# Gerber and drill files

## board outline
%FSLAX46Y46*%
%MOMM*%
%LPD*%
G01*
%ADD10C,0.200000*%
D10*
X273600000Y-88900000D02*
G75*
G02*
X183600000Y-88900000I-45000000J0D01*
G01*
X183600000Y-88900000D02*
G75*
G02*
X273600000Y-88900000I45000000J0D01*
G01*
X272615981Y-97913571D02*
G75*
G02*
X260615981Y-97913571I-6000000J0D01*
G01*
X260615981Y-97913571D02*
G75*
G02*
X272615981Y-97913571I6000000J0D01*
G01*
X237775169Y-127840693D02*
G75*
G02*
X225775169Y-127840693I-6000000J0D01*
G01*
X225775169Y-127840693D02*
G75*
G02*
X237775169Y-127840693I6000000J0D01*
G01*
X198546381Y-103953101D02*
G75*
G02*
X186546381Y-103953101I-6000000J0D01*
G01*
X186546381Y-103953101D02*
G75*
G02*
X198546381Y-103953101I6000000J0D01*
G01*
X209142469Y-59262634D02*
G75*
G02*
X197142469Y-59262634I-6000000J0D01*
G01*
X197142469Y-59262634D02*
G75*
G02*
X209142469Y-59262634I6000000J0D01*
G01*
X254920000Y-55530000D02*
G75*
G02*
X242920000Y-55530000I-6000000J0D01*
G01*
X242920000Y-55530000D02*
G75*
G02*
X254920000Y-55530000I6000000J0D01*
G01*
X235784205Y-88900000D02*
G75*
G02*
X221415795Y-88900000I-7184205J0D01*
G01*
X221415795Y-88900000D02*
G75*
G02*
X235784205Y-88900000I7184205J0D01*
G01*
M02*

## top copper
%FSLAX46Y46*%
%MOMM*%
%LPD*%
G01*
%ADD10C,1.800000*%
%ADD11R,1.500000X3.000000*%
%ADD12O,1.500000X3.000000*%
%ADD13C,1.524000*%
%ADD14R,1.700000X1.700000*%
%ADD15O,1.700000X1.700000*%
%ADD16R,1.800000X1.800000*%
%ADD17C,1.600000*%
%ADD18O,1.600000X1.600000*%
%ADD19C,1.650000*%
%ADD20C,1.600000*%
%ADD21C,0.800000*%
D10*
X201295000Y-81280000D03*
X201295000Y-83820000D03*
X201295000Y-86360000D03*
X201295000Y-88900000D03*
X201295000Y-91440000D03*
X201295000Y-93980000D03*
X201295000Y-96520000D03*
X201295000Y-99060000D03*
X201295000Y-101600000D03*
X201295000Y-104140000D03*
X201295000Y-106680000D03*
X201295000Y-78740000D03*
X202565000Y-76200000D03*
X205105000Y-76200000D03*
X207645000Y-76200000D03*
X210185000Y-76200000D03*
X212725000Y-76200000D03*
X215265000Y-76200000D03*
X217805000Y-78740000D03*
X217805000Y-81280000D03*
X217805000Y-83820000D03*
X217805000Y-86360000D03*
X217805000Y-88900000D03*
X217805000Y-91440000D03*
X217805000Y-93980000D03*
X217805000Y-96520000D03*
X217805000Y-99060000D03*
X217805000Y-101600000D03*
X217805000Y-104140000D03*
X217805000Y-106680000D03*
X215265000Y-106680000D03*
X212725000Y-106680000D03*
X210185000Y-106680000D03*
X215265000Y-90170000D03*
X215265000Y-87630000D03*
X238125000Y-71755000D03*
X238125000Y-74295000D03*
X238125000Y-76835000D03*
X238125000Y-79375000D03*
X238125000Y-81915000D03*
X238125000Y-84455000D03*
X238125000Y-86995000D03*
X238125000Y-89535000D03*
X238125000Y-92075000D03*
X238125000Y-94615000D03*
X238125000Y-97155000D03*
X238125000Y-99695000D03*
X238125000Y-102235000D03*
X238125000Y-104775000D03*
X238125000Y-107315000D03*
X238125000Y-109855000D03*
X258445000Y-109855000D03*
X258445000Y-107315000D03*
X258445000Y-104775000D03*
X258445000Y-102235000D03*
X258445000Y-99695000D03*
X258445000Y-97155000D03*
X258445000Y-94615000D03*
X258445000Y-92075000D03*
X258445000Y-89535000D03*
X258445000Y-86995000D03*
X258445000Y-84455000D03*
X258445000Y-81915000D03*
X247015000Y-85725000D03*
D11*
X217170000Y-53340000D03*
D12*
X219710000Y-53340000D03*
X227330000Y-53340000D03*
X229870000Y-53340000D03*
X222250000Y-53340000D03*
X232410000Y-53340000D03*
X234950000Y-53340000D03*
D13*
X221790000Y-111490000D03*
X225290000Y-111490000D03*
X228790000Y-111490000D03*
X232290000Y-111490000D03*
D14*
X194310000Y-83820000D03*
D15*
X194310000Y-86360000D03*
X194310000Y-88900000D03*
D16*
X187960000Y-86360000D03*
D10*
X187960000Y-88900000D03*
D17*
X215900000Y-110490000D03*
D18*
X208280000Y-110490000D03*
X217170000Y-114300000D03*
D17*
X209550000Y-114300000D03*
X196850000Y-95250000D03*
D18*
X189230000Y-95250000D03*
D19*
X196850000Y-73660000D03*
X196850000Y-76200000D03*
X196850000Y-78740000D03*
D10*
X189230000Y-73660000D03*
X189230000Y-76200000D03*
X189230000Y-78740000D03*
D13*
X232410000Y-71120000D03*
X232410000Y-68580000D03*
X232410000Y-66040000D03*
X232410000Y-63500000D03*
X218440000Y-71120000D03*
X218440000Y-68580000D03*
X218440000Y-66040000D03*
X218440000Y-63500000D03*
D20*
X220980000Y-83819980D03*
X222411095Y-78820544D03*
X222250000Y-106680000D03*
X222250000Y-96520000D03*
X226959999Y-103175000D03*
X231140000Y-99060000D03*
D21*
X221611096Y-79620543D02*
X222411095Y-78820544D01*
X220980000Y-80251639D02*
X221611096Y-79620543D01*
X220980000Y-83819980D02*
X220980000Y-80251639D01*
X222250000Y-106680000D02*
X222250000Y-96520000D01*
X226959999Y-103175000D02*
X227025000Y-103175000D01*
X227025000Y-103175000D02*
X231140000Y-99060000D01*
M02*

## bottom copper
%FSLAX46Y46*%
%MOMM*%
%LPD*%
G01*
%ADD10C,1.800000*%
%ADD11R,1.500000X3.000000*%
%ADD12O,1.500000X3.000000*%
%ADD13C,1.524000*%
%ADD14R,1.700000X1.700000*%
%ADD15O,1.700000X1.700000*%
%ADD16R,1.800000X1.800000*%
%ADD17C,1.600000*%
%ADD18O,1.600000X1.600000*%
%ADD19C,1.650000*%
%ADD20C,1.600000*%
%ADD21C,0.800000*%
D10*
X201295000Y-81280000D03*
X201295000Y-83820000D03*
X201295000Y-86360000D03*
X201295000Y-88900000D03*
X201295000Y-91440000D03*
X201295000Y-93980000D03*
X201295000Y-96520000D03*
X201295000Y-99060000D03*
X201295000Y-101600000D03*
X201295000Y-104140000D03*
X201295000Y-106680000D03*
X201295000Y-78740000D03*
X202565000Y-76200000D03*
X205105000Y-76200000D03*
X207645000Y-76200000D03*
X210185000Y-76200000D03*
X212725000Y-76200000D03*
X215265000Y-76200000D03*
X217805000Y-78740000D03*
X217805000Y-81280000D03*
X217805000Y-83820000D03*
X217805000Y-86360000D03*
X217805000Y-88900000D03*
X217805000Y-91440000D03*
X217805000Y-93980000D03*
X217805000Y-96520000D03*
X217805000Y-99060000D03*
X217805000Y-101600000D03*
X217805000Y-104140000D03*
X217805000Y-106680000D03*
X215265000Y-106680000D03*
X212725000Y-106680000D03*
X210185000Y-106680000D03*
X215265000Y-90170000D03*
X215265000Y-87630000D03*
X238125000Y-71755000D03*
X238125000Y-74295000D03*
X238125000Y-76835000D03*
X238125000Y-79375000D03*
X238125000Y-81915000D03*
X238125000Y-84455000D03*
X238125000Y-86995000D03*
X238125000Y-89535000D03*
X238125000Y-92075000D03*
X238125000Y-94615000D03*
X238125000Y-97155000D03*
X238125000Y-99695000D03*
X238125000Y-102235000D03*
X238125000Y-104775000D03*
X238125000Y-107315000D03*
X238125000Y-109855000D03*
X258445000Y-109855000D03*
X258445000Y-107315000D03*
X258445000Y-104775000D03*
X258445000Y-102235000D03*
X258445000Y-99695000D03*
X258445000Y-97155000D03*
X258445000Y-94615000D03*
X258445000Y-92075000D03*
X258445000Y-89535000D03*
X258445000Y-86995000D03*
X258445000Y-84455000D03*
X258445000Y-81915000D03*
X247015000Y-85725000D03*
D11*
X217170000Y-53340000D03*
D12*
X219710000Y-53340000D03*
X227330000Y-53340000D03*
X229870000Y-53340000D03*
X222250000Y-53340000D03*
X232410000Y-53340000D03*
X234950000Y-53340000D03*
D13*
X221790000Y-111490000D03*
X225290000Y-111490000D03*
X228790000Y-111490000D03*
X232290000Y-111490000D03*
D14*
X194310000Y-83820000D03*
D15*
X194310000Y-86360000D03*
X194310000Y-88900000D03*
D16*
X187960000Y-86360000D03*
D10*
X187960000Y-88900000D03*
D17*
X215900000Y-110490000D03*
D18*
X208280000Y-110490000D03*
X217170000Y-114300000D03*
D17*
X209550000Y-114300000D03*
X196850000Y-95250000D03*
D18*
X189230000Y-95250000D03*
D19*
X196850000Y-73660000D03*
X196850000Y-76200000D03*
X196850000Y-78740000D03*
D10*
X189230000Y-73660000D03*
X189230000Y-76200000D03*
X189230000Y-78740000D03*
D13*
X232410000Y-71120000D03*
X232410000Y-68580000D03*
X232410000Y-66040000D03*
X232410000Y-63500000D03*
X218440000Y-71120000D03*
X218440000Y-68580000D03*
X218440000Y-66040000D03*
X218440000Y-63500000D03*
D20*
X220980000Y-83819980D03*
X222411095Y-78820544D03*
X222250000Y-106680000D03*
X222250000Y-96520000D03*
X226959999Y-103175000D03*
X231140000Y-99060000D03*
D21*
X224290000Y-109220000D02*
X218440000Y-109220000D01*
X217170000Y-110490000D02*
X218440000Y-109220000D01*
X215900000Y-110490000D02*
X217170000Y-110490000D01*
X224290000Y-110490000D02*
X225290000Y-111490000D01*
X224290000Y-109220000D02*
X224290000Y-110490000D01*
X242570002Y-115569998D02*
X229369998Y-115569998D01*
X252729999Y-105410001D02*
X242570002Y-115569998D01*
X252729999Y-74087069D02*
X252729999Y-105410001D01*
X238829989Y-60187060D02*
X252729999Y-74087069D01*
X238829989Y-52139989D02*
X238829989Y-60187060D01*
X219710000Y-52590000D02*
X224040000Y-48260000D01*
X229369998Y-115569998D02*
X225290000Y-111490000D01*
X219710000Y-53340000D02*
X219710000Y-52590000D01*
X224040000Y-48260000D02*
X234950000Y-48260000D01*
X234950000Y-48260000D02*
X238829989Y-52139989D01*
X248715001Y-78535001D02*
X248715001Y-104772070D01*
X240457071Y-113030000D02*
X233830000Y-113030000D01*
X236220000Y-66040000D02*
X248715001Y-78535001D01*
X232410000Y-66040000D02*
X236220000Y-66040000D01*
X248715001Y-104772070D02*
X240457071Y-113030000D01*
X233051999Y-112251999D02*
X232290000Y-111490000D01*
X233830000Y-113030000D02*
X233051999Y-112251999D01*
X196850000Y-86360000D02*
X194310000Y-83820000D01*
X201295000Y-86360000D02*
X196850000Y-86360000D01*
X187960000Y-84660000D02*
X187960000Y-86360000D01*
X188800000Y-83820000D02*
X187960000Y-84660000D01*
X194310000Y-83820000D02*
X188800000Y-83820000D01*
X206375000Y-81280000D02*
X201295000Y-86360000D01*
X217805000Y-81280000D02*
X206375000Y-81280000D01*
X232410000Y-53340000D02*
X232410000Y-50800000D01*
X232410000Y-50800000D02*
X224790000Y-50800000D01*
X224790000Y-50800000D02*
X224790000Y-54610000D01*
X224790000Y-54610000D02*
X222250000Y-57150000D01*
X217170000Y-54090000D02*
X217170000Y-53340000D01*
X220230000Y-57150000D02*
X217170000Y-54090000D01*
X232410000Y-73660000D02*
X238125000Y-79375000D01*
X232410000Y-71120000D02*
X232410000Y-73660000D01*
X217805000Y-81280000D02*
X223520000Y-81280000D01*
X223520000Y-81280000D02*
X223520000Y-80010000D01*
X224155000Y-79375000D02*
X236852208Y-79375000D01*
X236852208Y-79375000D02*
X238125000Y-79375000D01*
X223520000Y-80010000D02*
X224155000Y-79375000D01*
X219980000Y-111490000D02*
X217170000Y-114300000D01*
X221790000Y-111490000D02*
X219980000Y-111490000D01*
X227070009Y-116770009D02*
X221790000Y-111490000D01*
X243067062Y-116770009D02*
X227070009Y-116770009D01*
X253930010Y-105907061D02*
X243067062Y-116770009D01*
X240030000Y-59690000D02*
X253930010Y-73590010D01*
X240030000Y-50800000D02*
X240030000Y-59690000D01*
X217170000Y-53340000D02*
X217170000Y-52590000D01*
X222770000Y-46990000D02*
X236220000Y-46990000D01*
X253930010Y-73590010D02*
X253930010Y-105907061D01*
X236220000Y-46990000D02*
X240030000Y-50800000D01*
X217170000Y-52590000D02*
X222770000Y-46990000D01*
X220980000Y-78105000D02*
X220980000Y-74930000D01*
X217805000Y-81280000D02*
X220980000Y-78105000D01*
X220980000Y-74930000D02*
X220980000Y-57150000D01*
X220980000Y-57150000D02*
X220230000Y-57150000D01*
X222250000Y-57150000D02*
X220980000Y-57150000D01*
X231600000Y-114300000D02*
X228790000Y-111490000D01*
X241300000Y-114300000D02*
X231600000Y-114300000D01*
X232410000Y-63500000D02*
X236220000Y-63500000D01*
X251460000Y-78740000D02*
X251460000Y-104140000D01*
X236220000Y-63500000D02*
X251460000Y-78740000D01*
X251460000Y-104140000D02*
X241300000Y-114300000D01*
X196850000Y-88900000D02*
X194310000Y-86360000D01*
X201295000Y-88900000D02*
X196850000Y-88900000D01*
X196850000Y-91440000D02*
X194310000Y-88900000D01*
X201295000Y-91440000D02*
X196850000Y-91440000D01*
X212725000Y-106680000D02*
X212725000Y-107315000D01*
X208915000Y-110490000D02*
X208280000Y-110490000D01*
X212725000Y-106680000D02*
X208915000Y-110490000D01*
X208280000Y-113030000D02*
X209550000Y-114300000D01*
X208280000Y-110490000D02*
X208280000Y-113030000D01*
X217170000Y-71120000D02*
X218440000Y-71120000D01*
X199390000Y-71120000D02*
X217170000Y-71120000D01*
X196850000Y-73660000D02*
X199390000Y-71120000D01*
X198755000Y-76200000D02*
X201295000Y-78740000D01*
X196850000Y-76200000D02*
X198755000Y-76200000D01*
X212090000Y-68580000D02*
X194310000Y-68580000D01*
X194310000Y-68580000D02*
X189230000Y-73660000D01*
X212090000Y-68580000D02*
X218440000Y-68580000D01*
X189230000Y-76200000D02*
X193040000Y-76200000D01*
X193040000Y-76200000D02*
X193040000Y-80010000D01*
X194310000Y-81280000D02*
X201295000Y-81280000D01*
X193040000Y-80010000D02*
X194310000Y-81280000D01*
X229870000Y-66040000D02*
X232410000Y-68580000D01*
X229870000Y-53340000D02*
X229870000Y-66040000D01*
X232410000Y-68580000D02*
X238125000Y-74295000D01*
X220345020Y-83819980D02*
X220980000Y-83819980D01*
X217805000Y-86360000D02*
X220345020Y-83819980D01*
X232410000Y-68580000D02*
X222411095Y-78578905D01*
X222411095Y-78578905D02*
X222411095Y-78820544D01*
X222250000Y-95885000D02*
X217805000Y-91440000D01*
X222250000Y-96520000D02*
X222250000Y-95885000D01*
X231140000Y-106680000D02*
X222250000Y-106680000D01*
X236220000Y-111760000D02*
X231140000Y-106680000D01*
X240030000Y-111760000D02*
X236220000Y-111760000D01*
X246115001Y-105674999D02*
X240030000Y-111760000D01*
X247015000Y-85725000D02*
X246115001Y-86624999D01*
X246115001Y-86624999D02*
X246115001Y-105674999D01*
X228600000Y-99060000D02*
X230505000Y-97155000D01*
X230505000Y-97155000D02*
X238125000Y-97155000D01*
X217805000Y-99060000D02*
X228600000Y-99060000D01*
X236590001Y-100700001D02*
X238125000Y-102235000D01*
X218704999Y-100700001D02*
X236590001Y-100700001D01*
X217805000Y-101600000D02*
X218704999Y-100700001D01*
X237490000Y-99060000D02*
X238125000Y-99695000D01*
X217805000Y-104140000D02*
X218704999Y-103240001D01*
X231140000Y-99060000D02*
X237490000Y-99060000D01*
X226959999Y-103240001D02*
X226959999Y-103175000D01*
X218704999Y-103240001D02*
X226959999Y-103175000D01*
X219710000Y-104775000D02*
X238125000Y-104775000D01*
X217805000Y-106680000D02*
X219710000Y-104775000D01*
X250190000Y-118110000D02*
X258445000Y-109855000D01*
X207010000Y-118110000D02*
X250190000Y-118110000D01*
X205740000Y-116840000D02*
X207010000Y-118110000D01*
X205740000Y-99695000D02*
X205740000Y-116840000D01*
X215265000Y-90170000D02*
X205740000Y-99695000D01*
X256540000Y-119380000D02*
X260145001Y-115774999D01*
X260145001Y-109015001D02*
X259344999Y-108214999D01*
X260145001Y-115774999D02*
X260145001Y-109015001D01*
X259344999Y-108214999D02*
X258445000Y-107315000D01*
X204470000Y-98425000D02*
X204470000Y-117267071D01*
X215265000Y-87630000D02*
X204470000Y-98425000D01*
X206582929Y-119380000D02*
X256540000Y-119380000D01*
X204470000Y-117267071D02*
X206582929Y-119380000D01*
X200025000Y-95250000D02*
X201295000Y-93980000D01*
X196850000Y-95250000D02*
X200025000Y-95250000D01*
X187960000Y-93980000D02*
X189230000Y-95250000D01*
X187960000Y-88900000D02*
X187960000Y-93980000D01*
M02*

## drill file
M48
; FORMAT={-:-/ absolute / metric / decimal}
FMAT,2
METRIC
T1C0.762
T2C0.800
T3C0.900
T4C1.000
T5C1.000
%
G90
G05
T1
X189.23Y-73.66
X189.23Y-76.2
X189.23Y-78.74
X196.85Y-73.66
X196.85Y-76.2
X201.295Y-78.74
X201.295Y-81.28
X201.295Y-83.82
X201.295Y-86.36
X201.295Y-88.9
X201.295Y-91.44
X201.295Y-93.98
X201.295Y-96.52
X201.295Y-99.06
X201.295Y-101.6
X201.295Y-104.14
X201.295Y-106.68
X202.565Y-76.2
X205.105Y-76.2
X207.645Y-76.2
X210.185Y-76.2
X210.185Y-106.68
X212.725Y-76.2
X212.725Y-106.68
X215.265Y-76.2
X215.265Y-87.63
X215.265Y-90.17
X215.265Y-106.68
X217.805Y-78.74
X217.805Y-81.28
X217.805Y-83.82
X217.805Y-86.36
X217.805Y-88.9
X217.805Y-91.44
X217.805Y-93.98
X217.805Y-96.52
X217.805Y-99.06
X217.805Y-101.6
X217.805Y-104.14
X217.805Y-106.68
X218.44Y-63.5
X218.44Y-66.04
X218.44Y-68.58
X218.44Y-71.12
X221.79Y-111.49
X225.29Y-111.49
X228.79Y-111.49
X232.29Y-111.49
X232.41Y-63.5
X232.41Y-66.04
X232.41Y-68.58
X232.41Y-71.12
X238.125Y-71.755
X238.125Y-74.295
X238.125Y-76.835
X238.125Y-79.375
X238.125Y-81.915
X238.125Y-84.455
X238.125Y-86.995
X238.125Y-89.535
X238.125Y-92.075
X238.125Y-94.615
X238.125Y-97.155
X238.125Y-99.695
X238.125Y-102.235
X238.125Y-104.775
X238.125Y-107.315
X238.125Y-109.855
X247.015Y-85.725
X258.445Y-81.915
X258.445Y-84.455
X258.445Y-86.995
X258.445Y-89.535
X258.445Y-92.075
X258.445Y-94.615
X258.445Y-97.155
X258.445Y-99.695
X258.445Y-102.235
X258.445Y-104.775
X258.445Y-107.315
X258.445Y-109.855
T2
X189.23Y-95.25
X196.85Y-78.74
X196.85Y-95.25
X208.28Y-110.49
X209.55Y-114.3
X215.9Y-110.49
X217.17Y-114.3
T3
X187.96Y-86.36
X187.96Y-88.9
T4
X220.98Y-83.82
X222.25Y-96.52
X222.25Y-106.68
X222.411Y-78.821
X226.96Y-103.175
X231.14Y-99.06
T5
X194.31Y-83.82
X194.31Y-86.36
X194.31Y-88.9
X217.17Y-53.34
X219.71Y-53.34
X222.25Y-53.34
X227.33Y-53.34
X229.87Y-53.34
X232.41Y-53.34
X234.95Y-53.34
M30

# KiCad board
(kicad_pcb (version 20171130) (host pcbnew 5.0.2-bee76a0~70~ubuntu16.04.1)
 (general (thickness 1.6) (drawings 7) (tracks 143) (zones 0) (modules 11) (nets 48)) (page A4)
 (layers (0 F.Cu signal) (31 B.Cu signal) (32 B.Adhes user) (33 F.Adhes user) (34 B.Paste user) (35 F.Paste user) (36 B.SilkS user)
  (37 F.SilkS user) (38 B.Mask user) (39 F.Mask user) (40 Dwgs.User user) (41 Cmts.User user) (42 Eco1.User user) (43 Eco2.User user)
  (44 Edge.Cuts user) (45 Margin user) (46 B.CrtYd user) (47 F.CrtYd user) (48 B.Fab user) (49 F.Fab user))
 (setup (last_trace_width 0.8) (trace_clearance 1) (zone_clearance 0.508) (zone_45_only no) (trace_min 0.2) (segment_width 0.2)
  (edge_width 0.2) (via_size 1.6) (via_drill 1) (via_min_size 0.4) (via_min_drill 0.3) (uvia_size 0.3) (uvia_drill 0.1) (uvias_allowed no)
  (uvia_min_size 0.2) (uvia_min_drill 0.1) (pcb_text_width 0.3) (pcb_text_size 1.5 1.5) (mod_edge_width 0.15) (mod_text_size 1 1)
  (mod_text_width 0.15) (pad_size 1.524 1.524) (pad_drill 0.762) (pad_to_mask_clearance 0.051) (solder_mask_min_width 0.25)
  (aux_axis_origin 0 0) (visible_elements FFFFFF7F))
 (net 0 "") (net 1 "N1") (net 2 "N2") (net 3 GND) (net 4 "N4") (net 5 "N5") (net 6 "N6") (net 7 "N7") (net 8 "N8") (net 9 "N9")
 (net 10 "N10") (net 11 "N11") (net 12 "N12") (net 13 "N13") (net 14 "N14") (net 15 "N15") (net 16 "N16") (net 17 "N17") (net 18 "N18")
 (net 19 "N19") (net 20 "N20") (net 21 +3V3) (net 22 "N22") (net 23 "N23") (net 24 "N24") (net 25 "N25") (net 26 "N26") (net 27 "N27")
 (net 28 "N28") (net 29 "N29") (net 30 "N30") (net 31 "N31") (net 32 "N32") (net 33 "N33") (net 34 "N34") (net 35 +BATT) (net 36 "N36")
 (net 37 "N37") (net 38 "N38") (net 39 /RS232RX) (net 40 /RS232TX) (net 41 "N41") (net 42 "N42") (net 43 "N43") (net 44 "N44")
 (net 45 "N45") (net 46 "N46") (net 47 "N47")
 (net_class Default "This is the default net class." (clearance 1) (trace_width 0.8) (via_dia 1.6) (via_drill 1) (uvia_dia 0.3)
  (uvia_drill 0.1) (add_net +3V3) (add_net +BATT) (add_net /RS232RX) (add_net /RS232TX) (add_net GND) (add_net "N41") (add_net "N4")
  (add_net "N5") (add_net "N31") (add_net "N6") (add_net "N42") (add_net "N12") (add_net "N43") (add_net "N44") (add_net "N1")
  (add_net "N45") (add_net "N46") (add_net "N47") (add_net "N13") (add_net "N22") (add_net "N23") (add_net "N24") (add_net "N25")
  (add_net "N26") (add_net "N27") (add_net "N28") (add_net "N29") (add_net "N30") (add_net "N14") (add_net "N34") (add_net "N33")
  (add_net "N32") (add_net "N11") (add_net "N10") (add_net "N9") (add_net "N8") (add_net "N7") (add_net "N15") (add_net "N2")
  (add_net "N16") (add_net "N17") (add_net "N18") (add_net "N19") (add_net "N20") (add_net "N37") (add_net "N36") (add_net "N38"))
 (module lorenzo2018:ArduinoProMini (layer F.Cu) (at 206.375 85.09)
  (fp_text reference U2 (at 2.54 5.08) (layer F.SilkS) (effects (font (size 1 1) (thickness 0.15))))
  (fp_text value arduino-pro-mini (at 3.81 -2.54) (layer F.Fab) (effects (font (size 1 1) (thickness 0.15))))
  (pad 34 thru_hole circle (at -5.08 -3.81) (size 1.8 1.8) (drill 0.762) (layers *.Cu *.Mask F.SilkS) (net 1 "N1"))
  (pad 33 thru_hole circle (at -5.08 -1.27) (size 1.8 1.8) (drill 0.762) (layers *.Cu *.Mask F.SilkS) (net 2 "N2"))
  (pad 32 thru_hole circle (at -5.08 1.27) (size 1.8 1.8) (drill 0.762) (layers *.Cu *.Mask F.SilkS) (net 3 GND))
  (pad 31 thru_hole circle (at -5.08 3.81) (size 1.8 1.8) (drill 0.762) (layers *.Cu *.Mask F.SilkS) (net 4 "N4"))
  (pad 30 thru_hole circle (at -5.08 6.35) (size 1.8 1.8) (drill 0.762) (layers *.Cu *.Mask F.SilkS) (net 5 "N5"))
  (pad 29 thru_hole circle (at -5.08 8.89) (size 1.8 1.8) (drill 0.762) (layers *.Cu *.Mask F.SilkS) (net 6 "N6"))
  (pad 28 thru_hole circle (at -5.08 11.43) (size 1.8 1.8) (drill 0.762) (layers *.Cu *.Mask F.SilkS) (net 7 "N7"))
  (pad 27 thru_hole circle (at -5.08 13.97) (size 1.8 1.8) (drill 0.762) (layers *.Cu *.Mask F.SilkS) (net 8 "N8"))
  (pad 26 thru_hole circle (at -5.08 16.51) (size 1.8 1.8) (drill 0.762) (layers *.Cu *.Mask F.SilkS) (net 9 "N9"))
  (pad 25 thru_hole circle (at -5.08 19.05) (size 1.8 1.8) (drill 0.762) (layers *.Cu *.Mask F.SilkS) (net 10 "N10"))
  (pad 24 thru_hole circle (at -5.08 21.59) (size 1.8 1.8) (drill 0.762) (layers *.Cu *.Mask F.SilkS) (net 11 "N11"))
  (pad 35 thru_hole circle (at -5.08 -6.35) (size 1.8 1.8) (drill 0.762) (layers *.Cu *.Mask F.SilkS) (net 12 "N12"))
  (pad 1 thru_hole circle (at -3.81 -8.89) (size 1.8 1.8) (drill 0.762) (layers *.Cu *.Mask F.SilkS) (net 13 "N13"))
  (pad 2 thru_hole circle (at -1.27 -8.89) (size 1.8 1.8) (drill 0.762) (layers *.Cu *.Mask F.SilkS) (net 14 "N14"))
  (pad 3 thru_hole circle (at 1.27 -8.89) (size 1.8 1.8) (drill 0.762) (layers *.Cu *.Mask F.SilkS) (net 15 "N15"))
  (pad 4 thru_hole circle (at 3.81 -8.89) (size 1.8 1.8) (drill 0.762) (layers *.Cu *.Mask F.SilkS) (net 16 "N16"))
  (pad 5 thru_hole circle (at 6.35 -8.89) (size 1.8 1.8) (drill 0.762) (layers *.Cu *.Mask F.SilkS) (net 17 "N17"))
  (pad 6 thru_hole circle (at 8.89 -8.89) (size 1.8 1.8) (drill 0.762) (layers *.Cu *.Mask F.SilkS) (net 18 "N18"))
  (pad 7 thru_hole circle (at 11.43 -6.35) (size 1.8 1.8) (drill 0.762) (layers *.Cu *.Mask F.SilkS) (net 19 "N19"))
  (pad 8 thru_hole circle (at 11.43 -3.81) (size 1.8 1.8) (drill 0.762) (layers *.Cu *.Mask F.SilkS) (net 3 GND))
  (pad 9 thru_hole circle (at 11.43 -1.27) (size 1.8 1.8) (drill 0.762) (layers *.Cu *.Mask F.SilkS) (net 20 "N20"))
  (pad 10 thru_hole circle (at 11.43 1.27) (size 1.8 1.8) (drill 0.762) (layers *.Cu *.Mask F.SilkS) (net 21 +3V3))
  (pad 11 thru_hole circle (at 11.43 3.81) (size 1.8 1.8) (drill 0.762) (layers *.Cu *.Mask F.SilkS) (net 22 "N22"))
  (pad 12 thru_hole circle (at 11.43 6.35) (size 1.8 1.8) (drill 0.762) (layers *.Cu *.Mask F.SilkS) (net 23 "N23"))
  (pad 13 thru_hole circle (at 11.43 8.89) (size 1.8 1.8) (drill 0.762) (layers *.Cu *.Mask F.SilkS) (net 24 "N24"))
  (pad 14 thru_hole circle (at 11.43 11.43) (size 1.8 1.8) (drill 0.762) (layers *.Cu *.Mask F.SilkS) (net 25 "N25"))
  (pad 15 thru_hole circle (at 11.43 13.97) (size 1.8 1.8) (drill 0.762) (layers *.Cu *.Mask F.SilkS) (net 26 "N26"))
  (pad 16 thru_hole circle (at 11.43 16.51) (size 1.8 1.8) (drill 0.762) (layers *.Cu *.Mask F.SilkS) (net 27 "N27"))
  (pad 17 thru_hole circle (at 11.43 19.05) (size 1.8 1.8) (drill 0.762) (layers *.Cu *.Mask F.SilkS) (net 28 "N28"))
  (pad 18 thru_hole circle (at 11.43 21.59) (size 1.8 1.8) (drill 0.762) (layers *.Cu *.Mask F.SilkS) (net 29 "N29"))
  (pad 19 thru_hole circle (at 8.89 21.59) (size 1.8 1.8) (drill 0.762) (layers *.Cu *.Mask F.SilkS) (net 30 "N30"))
  (pad 20 thru_hole circle (at 6.35 21.59) (size 1.8 1.8) (drill 0.762) (layers *.Cu *.Mask F.SilkS) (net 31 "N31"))
  (pad 23 thru_hole circle (at 3.81 21.59) (size 1.8 1.8) (drill 0.762) (layers *.Cu *.Mask F.SilkS) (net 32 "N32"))
  (pad 22 thru_hole circle (at 8.89 5.08) (size 1.8 1.8) (drill 0.762) (layers *.Cu *.Mask F.SilkS) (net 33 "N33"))
  (pad 21 thru_hole circle (at 8.89 2.54) (size 1.8 1.8) (drill 0.762) (layers *.Cu *.Mask F.SilkS) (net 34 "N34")))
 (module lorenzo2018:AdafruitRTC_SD (layer F.Cu) (at 240.665 75.565)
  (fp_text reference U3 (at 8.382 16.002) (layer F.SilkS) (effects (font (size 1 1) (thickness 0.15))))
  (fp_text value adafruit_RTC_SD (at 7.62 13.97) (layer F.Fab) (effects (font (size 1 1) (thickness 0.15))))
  (pad 1 thru_hole circle (at -2.54 -3.81) (size 1.8 1.8) (drill 0.762) (layers *.Cu *.Mask F.SilkS))
  (pad 2 thru_hole circle (at -2.54 -1.27) (size 1.8 1.8) (drill 0.762) (layers *.Cu *.Mask F.SilkS) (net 21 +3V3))
  (pad 3 thru_hole circle (at -2.54 1.27) (size 1.8 1.8) (drill 0.762) (layers *.Cu *.Mask F.SilkS))
  (pad 4 thru_hole circle (at -2.54 3.81) (size 1.8 1.8) (drill 0.762) (layers *.Cu *.Mask F.SilkS) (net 3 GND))
  (pad 5 thru_hole circle (at -2.54 6.35) (size 1.8 1.8) (drill 0.762) (layers *.Cu *.Mask F.SilkS))
  (pad 6 thru_hole circle (at -2.54 8.89) (size 1.8 1.8) (drill 0.762) (layers *.Cu *.Mask F.SilkS))
  (pad 7 thru_hole circle (at -2.54 11.43) (size 1.8 1.8) (drill 0.762) (layers *.Cu *.Mask F.SilkS))
  (pad 8 thru_hole circle (at -2.54 13.97) (size 1.8 1.8) (drill 0.762) (layers *.Cu *.Mask F.SilkS))
  (pad 9 thru_hole circle (at -2.54 16.51) (size 1.8 1.8) (drill 0.762) (layers *.Cu *.Mask F.SilkS))
  (pad 10 thru_hole circle (at -2.54 19.05) (size 1.8 1.8) (drill 0.762) (layers *.Cu *.Mask F.SilkS))
  (pad 11 thru_hole circle (at -2.54 21.59) (size 1.8 1.8) (drill 0.762) (layers *.Cu *.Mask F.SilkS) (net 26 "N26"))
  (pad 12 thru_hole circle (at -2.54 24.13) (size 1.8 1.8) (drill 0.762) (layers *.Cu *.Mask F.SilkS) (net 28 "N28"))
  (pad 13 thru_hole circle (at -2.54 26.67) (size 1.8 1.8) (drill 0.762) (layers *.Cu *.Mask F.SilkS) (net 27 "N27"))
  (pad 14 thru_hole circle (at -2.54 29.21) (size 1.8 1.8) (drill 0.762) (layers *.Cu *.Mask F.SilkS) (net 29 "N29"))
  (pad 15 thru_hole circle (at -2.54 31.75) (size 1.8 1.8) (drill 0.762) (layers *.Cu *.Mask F.SilkS))
  (pad 16 thru_hole circle (at -2.54 34.29) (size 1.8 1.8) (drill 0.762) (layers *.Cu *.Mask F.SilkS))
  (pad 17 thru_hole circle (at 17.78 34.29) (size 1.8 1.8) (drill 0.762) (layers *.Cu *.Mask F.SilkS) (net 33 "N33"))
  (pad 18 thru_hole circle (at 17.78 31.75) (size 1.8 1.8) (drill 0.762) (layers *.Cu *.Mask F.SilkS) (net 34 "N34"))
  (pad 19 thru_hole circle (at 17.78 29.21) (size 1.8 1.8) (drill 0.762) (layers *.Cu *.Mask F.SilkS))
  (pad 20 thru_hole circle (at 17.78 26.67) (size 1.8 1.8) (drill 0.762) (layers *.Cu *.Mask F.SilkS))
  (pad 21 thru_hole circle (at 17.78 24.13) (size 1.8 1.8) (drill 0.762) (layers *.Cu *.Mask F.SilkS))
  (pad 22 thru_hole circle (at 17.78 21.59) (size 1.8 1.8) (drill 0.762) (layers *.Cu *.Mask F.SilkS))
  (pad 23 thru_hole circle (at 17.78 19.05) (size 1.8 1.8) (drill 0.762) (layers *.Cu *.Mask F.SilkS))
  (pad 24 thru_hole circle (at 17.78 16.51) (size 1.8 1.8) (drill 0.762) (layers *.Cu *.Mask F.SilkS))
  (pad 25 thru_hole circle (at 17.78 13.97) (size 1.8 1.8) (drill 0.762) (layers *.Cu *.Mask F.SilkS))
  (pad 26 thru_hole circle (at 17.78 11.43) (size 1.8 1.8) (drill 0.762) (layers *.Cu *.Mask F.SilkS))
  (pad 27 thru_hole circle (at 17.78 8.89) (size 1.8 1.8) (drill 0.762) (layers *.Cu *.Mask F.SilkS))
  (pad 28 thru_hole circle (at 17.78 6.35) (size 1.8 1.8) (drill 0.762) (layers *.Cu *.Mask F.SilkS))
  (pad 29 thru_hole circle (at 6.35 10.16) (size 1.8 1.8) (drill 0.762) (layers *.Cu *.Mask F.SilkS) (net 23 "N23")))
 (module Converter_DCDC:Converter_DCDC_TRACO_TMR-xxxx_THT (layer F.Cu) (at 217.17 53.34)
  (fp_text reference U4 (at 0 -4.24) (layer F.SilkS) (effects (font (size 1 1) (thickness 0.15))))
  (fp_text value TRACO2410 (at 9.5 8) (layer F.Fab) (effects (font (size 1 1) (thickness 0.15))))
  (pad 1 thru_hole rect (at 0 0) (size 1.5 3) (drill 1) (layers *.Cu *.Mask) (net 3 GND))
  (pad 2 thru_hole oval (at 2.54 0) (size 1.5 3) (drill 1) (layers *.Cu *.Mask) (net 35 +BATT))
  (pad 5 thru_hole oval (at 10.16 0) (size 1.5 3) (drill 1) (layers *.Cu *.Mask) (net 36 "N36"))
  (pad 6 thru_hole oval (at 12.7 0) (size 1.5 3) (drill 1) (layers *.Cu *.Mask) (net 21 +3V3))
  (pad 3 thru_hole oval (at 5.08 0) (size 1.5 3) (drill 1) (layers *.Cu *.Mask) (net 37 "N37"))
  (pad 7 thru_hole oval (at 15.24 0) (size 1.5 3) (drill 1) (layers *.Cu *.Mask) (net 3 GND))
  (pad 8 thru_hole oval (at 17.78 0) (size 1.5 3) (drill 1) (layers *.Cu *.Mask) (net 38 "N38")))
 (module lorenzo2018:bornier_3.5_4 (layer F.Cu) (at 224.79 110.49)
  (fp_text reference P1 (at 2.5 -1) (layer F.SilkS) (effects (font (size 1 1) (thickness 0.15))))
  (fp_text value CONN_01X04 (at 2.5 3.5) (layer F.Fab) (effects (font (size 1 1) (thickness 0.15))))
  (pad 1 thru_hole circle (at -3 1) (size 1.524 1.524) (drill 0.762) (layers *.Cu *.Mask) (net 3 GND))
  (pad 2 thru_hole circle (at 0.5 1) (size 1.524 1.524) (drill 0.762) (layers *.Cu *.Mask) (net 35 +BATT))
  (pad 3 thru_hole circle (at 4 1) (size 1.524 1.524) (drill 0.762) (layers *.Cu *.Mask) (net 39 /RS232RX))
  (pad 4 thru_hole circle (at 7.5 1) (size 1.524 1.524) (drill 0.762) (layers *.Cu *.Mask) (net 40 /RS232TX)))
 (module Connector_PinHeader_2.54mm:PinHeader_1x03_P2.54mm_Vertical (layer F.Cu) (at 194.31 83.82)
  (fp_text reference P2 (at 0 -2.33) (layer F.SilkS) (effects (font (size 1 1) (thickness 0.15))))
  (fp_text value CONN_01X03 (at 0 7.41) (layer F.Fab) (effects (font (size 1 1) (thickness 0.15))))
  (pad 1 thru_hole rect (at 0 0) (size 1.7 1.7) (drill 1) (layers *.Cu *.Mask) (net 3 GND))
  (pad 2 thru_hole oval (at 0 2.54) (size 1.7 1.7) (drill 1) (layers *.Cu *.Mask) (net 4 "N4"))
  (pad 3 thru_hole oval (at 0 5.08) (size 1.7 1.7) (drill 1) (layers *.Cu *.Mask) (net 5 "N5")))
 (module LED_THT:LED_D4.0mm (layer F.Cu) (at 187.96 86.36 270)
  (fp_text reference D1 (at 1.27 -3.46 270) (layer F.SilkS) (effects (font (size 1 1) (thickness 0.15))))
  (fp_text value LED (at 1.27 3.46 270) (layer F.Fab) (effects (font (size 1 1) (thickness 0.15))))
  (pad 1 thru_hole rect (at 0 0 270) (size 1.8 1.8) (drill 0.9) (layers *.Cu *.Mask) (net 3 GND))
  (pad 2 thru_hole circle (at 2.54 0 270) (size 1.8 1.8) (drill 0.9) (layers *.Cu *.Mask) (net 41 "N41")))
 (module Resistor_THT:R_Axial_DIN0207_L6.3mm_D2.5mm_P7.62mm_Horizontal (layer F.Cu) (at 215.9 110.49 180)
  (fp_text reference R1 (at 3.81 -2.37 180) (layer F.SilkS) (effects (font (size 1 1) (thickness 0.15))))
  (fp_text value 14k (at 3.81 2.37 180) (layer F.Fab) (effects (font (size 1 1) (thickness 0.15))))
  (pad 1 thru_hole circle (at 0 0 180) (size 1.6 1.6) (drill 0.8) (layers *.Cu *.Mask) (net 35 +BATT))
  (pad 2 thru_hole oval (at 7.62 0 180) (size 1.6 1.6) (drill 0.8) (layers *.Cu *.Mask) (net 31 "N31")))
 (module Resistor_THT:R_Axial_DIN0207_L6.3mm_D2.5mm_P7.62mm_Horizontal (layer F.Cu) (at 209.55 114.3)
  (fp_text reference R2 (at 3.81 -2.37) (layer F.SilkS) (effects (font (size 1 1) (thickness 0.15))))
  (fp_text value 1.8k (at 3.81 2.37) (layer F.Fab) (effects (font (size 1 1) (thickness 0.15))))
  (pad 2 thru_hole oval (at 7.62 0) (size 1.6 1.6) (drill 0.8) (layers *.Cu *.Mask) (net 3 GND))
  (pad 1 thru_hole circle (at 0 0) (size 1.6 1.6) (drill 0.8) (layers *.Cu *.Mask) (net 31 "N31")))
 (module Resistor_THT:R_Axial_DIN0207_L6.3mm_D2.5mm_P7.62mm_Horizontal (layer F.Cu) (at 196.85 95.25 180)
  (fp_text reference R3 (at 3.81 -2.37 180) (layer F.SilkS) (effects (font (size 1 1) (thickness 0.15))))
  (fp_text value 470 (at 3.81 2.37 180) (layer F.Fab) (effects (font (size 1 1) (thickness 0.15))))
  (pad 1 thru_hole circle (at 0 0 180) (size 1.6 1.6) (drill 0.8) (layers *.Cu *.Mask) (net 6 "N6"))
  (pad 2 thru_hole oval (at 7.62 0 180) (size 1.6 1.6) (drill 0.8) (layers *.Cu *.Mask) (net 41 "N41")))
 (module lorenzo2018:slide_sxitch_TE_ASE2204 (layer F.Cu) (at 193.04 77.47 270)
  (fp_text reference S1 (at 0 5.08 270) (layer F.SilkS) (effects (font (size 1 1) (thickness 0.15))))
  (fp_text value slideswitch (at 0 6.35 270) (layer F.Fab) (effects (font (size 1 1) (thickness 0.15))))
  (pad 1 thru_hole circle (at -3.81 -3.81 270) (size 1.65 1.65) (drill 0.762) (layers *.Cu *.Mask) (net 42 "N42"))
  (pad 2 thru_hole circle (at -1.27 -3.81 270) (size 1.65 1.65) (drill 0.762) (layers *.Cu *.Mask) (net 12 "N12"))
  (pad 3 thru_hole circle (at 1.27 -3.81 270) (size 1.65 1.65) (drill 0.8) (layers *.Cu *.Mask) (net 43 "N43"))
  (pad 4 thru_hole circle (at -3.81 3.81 270) (size 1.8 1.8) (drill 0.762) (layers *.Cu *.Mask) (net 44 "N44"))
  (pad 5 thru_hole circle (at -1.27 3.81 270) (size 1.8 1.8) (drill 0.762) (layers *.Cu *.Mask) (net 1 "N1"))
  (pad 6 thru_hole circle (at 1.27 3.81 270) (size 1.8 1.8) (drill 0.762) (layers *.Cu *.Mask) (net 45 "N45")))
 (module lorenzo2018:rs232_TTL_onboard (layer F.Cu) (at 222.25 71.12 180)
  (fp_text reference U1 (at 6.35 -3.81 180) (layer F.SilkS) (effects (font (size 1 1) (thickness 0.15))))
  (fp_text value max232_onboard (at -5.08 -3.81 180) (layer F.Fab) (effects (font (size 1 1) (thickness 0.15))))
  (pad 1 thru_hole circle (at -10.16 0 180) (size 1.524 1.524) (drill 0.762) (layers *.Cu *.Mask) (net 3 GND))
  (pad 2 thru_hole circle (at -10.16 2.54 180) (size 1.524 1.524) (drill 0.762) (layers *.Cu *.Mask) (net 21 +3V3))
  (pad 3 thru_hole circle (at -10.16 5.08 180) (size 1.524 1.524) (drill 0.762) (layers *.Cu *.Mask) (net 40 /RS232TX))
  (pad 4 thru_hole circle (at -10.16 7.62 180) (size 1.524 1.524) (drill 0.762) (layers *.Cu *.Mask) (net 39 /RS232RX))
  (pad 5 thru_hole circle (at 3.81 0 180) (size 1.524 1.524) (drill 0.762) (layers *.Cu *.Mask) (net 42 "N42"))
  (pad 6 thru_hole circle (at 3.81 2.54 180) (size 1.524 1.524) (drill 0.762) (layers *.Cu *.Mask) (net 44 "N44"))
  (pad 7 thru_hole circle (at 3.81 5.08 180) (size 1.524 1.524) (drill 0.762) (layers *.Cu *.Mask) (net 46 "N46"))
  (pad 8 thru_hole circle (at 3.81 7.62 180) (size 1.524 1.524) (drill 0.762) (layers *.Cu *.Mask) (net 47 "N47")))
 (gr_circle (center 228.6 88.9) (end 273.6 88.9) (layer Edge.Cuts) (width 0.2))
 (gr_circle (center 266.615981 97.913571) (end 272.615981 97.913571) (layer Edge.Cuts) (width 0.2))
 (gr_circle (center 231.775169 127.840693) (end 237.775169 127.840693) (layer Edge.Cuts) (width 0.2))
 (gr_circle (center 192.546381 103.953101) (end 198.546381 103.953101) (layer Edge.Cuts) (width 0.2))
 (gr_circle (center 203.142469 59.262634) (end 209.142469 59.262634) (layer Edge.Cuts) (width 0.2))
 (gr_circle (center 248.92 55.53) (end 254.92 55.53) (layer Edge.Cuts) (width 0.2))
 (gr_circle (center 228.6 88.9) (end 235.784205 88.9) (layer Edge.Cuts) (width 0.2))
 (segment (start 224.29 109.22) (end 218.44 109.22) (width 0.8) (layer B.Cu) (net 35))
 (segment (start 217.17 110.49) (end 218.44 109.22) (width 0.8) (layer B.Cu) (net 35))
 (segment (start 215.9 110.49) (end 217.17 110.49) (width 0.8) (layer B.Cu) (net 35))
 (segment (start 224.29 110.49) (end 225.29 111.49) (width 0.8) (layer B.Cu) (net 35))
 (segment (start 224.29 109.22) (end 224.29 110.49) (width 0.8) (layer B.Cu) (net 35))
 (segment (start 242.570002 115.569998) (end 229.369998 115.569998) (width 0.8) (layer B.Cu) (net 35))
 (segment (start 252.729999 105.410001) (end 242.570002 115.569998) (width 0.8) (layer B.Cu) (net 35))
 (segment (start 252.729999 74.087069) (end 252.729999 105.410001) (width 0.8) (layer B.Cu) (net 35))
 (segment (start 238.829989 60.18706) (end 252.729999 74.087069) (width 0.8) (layer B.Cu) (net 35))
 (segment (start 238.829989 52.139989) (end 238.829989 60.18706) (width 0.8) (layer B.Cu) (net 35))
 (segment (start 219.71 52.59) (end 224.04 48.26) (width 0.8) (layer B.Cu) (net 35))
 (segment (start 229.369998 115.569998) (end 225.29 111.49) (width 0.8) (layer B.Cu) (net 35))
 (segment (start 219.71 53.34) (end 219.71 52.59) (width 0.8) (layer B.Cu) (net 35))
 (segment (start 224.04 48.26) (end 234.95 48.26) (width 0.8) (layer B.Cu) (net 35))
 (segment (start 234.95 48.26) (end 238.829989 52.139989) (width 0.8) (layer B.Cu) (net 35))
 (segment (start 248.715001 78.535001) (end 248.715001 104.77207) (width 0.8) (layer B.Cu) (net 40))
 (segment (start 240.457071 113.03) (end 233.83 113.03) (width 0.8) (layer B.Cu) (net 40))
 (segment (start 236.22 66.04) (end 248.715001 78.535001) (width 0.8) (layer B.Cu) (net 40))
 (segment (start 232.41 66.04) (end 236.22 66.04) (width 0.8) (layer B.Cu) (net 40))
 (segment (start 248.715001 104.77207) (end 240.457071 113.03) (width 0.8) (layer B.Cu) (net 40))
 (segment (start 233.051999 112.251999) (end 232.29 111.49) (width 0.8) (layer B.Cu) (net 40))
 (segment (start 233.83 113.03) (end 233.051999 112.251999) (width 0.8) (layer B.Cu) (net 40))
 (segment (start 196.85 86.36) (end 194.31 83.82) (width 0.8) (layer B.Cu) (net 3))
 (segment (start 201.295 86.36) (end 196.85 86.36) (width 0.8) (layer B.Cu) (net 3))
 (segment (start 187.96 84.66) (end 187.96 86.36) (width 0.8) (layer B.Cu) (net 3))
 (segment (start 188.8 83.82) (end 187.96 84.66) (width 0.8) (layer B.Cu) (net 3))
 (segment (start 194.31 83.82) (end 188.8 83.82) (width 0.8) (layer B.Cu) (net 3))
 (segment (start 206.375 81.28) (end 201.295 86.36) (width 0.8) (layer B.Cu) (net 3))
 (segment (start 217.805 81.28) (end 206.375 81.28) (width 0.8) (layer B.Cu) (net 3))
 (segment (start 232.41 53.34) (end 232.41 50.8) (width 0.8) (layer B.Cu) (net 3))
 (segment (start 232.41 50.8) (end 224.79 50.8) (width 0.8) (layer B.Cu) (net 3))
 (segment (start 224.79 50.8) (end 224.79 54.61) (width 0.8) (layer B.Cu) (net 3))
 (segment (start 224.79 54.61) (end 222.25 57.15) (width 0.8) (layer B.Cu) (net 3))
 (segment (start 217.17 54.09) (end 217.17 53.34) (width 0.8) (layer B.Cu) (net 3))
 (segment (start 220.23 57.15) (end 217.17 54.09) (width 0.8) (layer B.Cu) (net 3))
 (segment (start 232.41 73.66) (end 238.125 79.375) (width 0.8) (layer B.Cu) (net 3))
 (segment (start 232.41 71.12) (end 232.41 73.66) (width 0.8) (layer B.Cu) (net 3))
 (segment (start 217.805 81.28) (end 223.52 81.28) (width 0.8) (layer B.Cu) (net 3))
 (segment (start 223.52 81.28) (end 223.52 80.01) (width 0.8) (layer B.Cu) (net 3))
 (segment (start 224.155 79.375) (end 236.852208 79.375) (width 0.8) (layer B.Cu) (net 3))
 (segment (start 236.852208 79.375) (end 238.125 79.375) (width 0.8) (layer B.Cu) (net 3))
 (segment (start 223.52 80.01) (end 224.155 79.375) (width 0.8) (layer B.Cu) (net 3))
 (segment (start 219.98 111.49) (end 217.17 114.3) (width 0.8) (layer B.Cu) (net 3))
 (segment (start 221.79 111.49) (end 219.98 111.49) (width 0.8) (layer B.Cu) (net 3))
 (segment (start 227.070009 116.770009) (end 221.79 111.49) (width 0.8) (layer B.Cu) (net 3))
 (segment (start 243.067062 116.770009) (end 227.070009 116.770009) (width 0.8) (layer B.Cu) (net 3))
 (segment (start 253.93001 105.907061) (end 243.067062 116.770009) (width 0.8) (layer B.Cu) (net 3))
 (segment (start 240.03 59.69) (end 253.93001 73.59001) (width 0.8) (layer B.Cu) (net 3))
 (segment (start 240.03 50.8) (end 240.03 59.69) (width 0.8) (layer B.Cu) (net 3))
 (segment (start 217.17 53.34) (end 217.17 52.59) (width 0.8) (layer B.Cu) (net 3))
 (segment (start 222.77 46.99) (end 236.22 46.99) (width 0.8) (layer B.Cu) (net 3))
 (segment (start 253.93001 73.59001) (end 253.93001 105.907061) (width 0.8) (layer B.Cu) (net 3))
 (segment (start 236.22 46.99) (end 240.03 50.8) (width 0.8) (layer B.Cu) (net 3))
 (segment (start 217.17 52.59) (end 222.77 46.99) (width 0.8) (layer B.Cu) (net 3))
 (segment (start 220.98 78.105) (end 220.98 74.93) (width 0.8) (layer B.Cu) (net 3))
 (segment (start 217.805 81.28) (end 220.98 78.105) (width 0.8) (layer B.Cu) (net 3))
 (segment (start 220.98 74.93) (end 220.98 57.15) (width 0.8) (layer B.Cu) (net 3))
 (segment (start 220.98 57.15) (end 220.23 57.15) (width 0.8) (layer B.Cu) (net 3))
 (segment (start 222.25 57.15) (end 220.98 57.15) (width 0.8) (layer B.Cu) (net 3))
 (segment (start 231.6 114.3) (end 228.79 111.49) (width 0.8) (layer B.Cu) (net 39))
 (segment (start 241.3 114.3) (end 231.6 114.3) (width 0.8) (layer B.Cu) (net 39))
 (segment (start 232.41 63.5) (end 236.22 63.5) (width 0.8) (layer B.Cu) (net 39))
 (segment (start 251.46 78.74) (end 251.46 104.14) (width 0.8) (layer B.Cu) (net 39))
 (segment (start 236.22 63.5) (end 251.46 78.74) (width 0.8) (layer B.Cu) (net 39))
 (segment (start 251.46 104.14) (end 241.3 114.3) (width 0.8) (layer B.Cu) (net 39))
 (segment (start 196.85 88.9) (end 194.31 86.36) (width 0.8) (layer B.Cu) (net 4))
 (segment (start 201.295 88.9) (end 196.85 88.9) (width 0.8) (layer B.Cu) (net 4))
 (segment (start 196.85 91.44) (end 194.31 88.9) (width 0.8) (layer B.Cu) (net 5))
 (segment (start 201.295 91.44) (end 196.85 91.44) (width 0.8) (layer B.Cu) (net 5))
 (segment (start 212.725 106.68) (end 212.725 107.315) (width 0.8) (layer B.Cu) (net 31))
 (segment (start 208.915 110.49) (end 208.28 110.49) (width 0.8) (layer B.Cu) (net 31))
 (segment (start 212.725 106.68) (end 208.915 110.49) (width 0.8) (layer B.Cu) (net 31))
 (segment (start 208.28 113.03) (end 209.55 114.3) (width 0.8) (layer B.Cu) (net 31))
 (segment (start 208.28 110.49) (end 208.28 113.03) (width 0.8) (layer B.Cu) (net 31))
 (segment (start 217.17 71.12) (end 218.44 71.12) (width 0.8) (layer B.Cu) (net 42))
 (segment (start 199.39 71.12) (end 217.17 71.12) (width 0.8) (layer B.Cu) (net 42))
 (segment (start 196.85 73.66) (end 199.39 71.12) (width 0.8) (layer B.Cu) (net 42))
 (segment (start 198.755 76.2) (end 201.295 78.74) (width 0.8) (layer B.Cu) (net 12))
 (segment (start 196.85 76.2) (end 198.755 76.2) (width 0.8) (layer B.Cu) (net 12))
 (segment (start 212.09 68.58) (end 194.31 68.58) (width 0.8) (layer B.Cu) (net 44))
 (segment (start 194.31 68.58) (end 189.23 73.66) (width 0.8) (layer B.Cu) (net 44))
 (segment (start 212.09 68.58) (end 218.44 68.58) (width 0.8) (layer B.Cu) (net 44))
 (segment (start 189.23 76.2) (end 193.04 76.2) (width 0.8) (layer B.Cu) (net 1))
 (segment (start 193.04 76.2) (end 193.04 80.01) (width 0.8) (layer B.Cu) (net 1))
 (segment (start 194.31 81.28) (end 201.295 81.28) (width 0.8) (layer B.Cu) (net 1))
 (segment (start 193.04 80.01) (end 194.31 81.28) (width 0.8) (layer B.Cu) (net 1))
 (segment (start 229.87 66.04) (end 232.41 68.58) (width 0.8) (layer B.Cu) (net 21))
 (segment (start 229.87 53.34) (end 229.87 66.04) (width 0.8) (layer B.Cu) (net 21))
 (segment (start 232.41 68.58) (end 238.125 74.295) (width 0.8) (layer B.Cu) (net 21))
 (via (at 220.98 83.81998) (size 1.6) (drill 1) (layers F.Cu B.Cu) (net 21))
 (segment (start 220.34502 83.81998) (end 220.98 83.81998) (width 0.8) (layer B.Cu) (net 21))
 (segment (start 217.805 86.36) (end 220.34502 83.81998) (width 0.8) (layer B.Cu) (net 21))
 (segment (start 232.41 68.58) (end 222.411095 78.578905) (width 0.8) (layer B.Cu) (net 21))
 (via (at 222.411095 78.820544) (size 1.6) (drill 1) (layers F.Cu B.Cu) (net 21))
 (segment (start 221.611096 79.620543) (end 222.411095 78.820544) (width 0.8) (layer F.Cu) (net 21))
 (segment (start 220.98 80.251639) (end 221.611096 79.620543) (width 0.8) (layer F.Cu) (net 21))
 (segment (start 220.98 83.81998) (end 220.98 80.251639) (width 0.8) (layer F.Cu) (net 21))
 (segment (start 222.411095 78.578905) (end 222.411095 78.820544) (width 0.8) (layer B.Cu) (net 21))
 (via (at 222.25 106.68) (size 1.6) (drill 1) (layers F.Cu B.Cu) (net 23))
 (segment (start 222.25 106.68) (end 222.25 96.52) (width 0.8) (layer F.Cu) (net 23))
 (via (at 222.25 96.52) (size 1.6) (drill 1) (layers F.Cu B.Cu) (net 23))
 (segment (start 222.25 95.885) (end 217.805 91.44) (width 0.8) (layer B.Cu) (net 23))
 (segment (start 222.25 96.52) (end 222.25 95.885) (width 0.8) (layer B.Cu) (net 23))
 (segment (start 231.14 106.68) (end 222.25 106.68) (width 0.8) (layer B.Cu) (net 23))
 (segment (start 236.22 111.76) (end 231.14 106.68) (width 0.8) (layer B.Cu) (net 23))
 (segment (start 240.03 111.76) (end 236.22 111.76) (width 0.8) (layer B.Cu) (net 23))
 (segment (start 246.115001 105.674999) (end 240.03 111.76) (width 0.8) (layer B.Cu) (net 23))
 (segment (start 247.015 85.725) (end 246.115001 86.624999) (width 0.8) (layer B.Cu) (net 23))
 (segment (start 246.115001 86.624999) (end 246.115001 105.674999) (width 0.8) (layer B.Cu) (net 23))
 (segment (start 228.6 99.06) (end 230.505 97.155) (width 0.8) (layer B.Cu) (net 26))
 (segment (start 230.505 97.155) (end 238.125 97.155) (width 0.8) (layer B.Cu) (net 26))
 (segment (start 217.805 99.06) (end 228.6 99.06) (width 0.8) (layer B.Cu) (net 26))
 (segment (start 236.590001 100.700001) (end 238.125 102.235) (width 0.8) (layer B.Cu) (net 27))
 (segment (start 218.704999 100.700001) (end 236.590001 100.700001) (width 0.8) (layer B.Cu) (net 27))
 (segment (start 217.805 101.6) (end 218.704999 100.700001) (width 0.8) (layer B.Cu) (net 27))
 (segment (start 237.49 99.06) (end 238.125 99.695) (width 0.8) (layer B.Cu) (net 28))
 (segment (start 217.805 104.14) (end 218.704999 103.240001) (width 0.8) (layer B.Cu) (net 28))
 (segment (start 231.14 99.06) (end 237.49 99.06) (width 0.8) (layer B.Cu) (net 28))
 (via (at 226.959999 103.175) (size 1.6) (drill 1) (layers F.Cu B.Cu) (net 28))
 (segment (start 226.959999 103.240001) (end 226.959999 103.175) (width 0.8) (layer B.Cu) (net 28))
 (segment (start 218.704999 103.240001) (end 226.959999 103.175) (width 0.8) (layer B.Cu) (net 28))
 (segment (start 226.959999 103.175) (end 227.025 103.175) (width 0.8) (layer F.Cu) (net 28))
 (via (at 231.14 99.06) (size 1.6) (drill 1) (layers F.Cu B.Cu) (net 28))
 (segment (start 227.025 103.175) (end 231.14 99.06) (width 0.8) (layer F.Cu) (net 28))
 (segment (start 219.71 104.775) (end 238.125 104.775) (width 0.8) (layer B.Cu) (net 29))
 (segment (start 217.805 106.68) (end 219.71 104.775) (width 0.8) (layer B.Cu) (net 29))
 (segment (start 250.19 118.11) (end 258.445 109.855) (width 0.8) (layer B.Cu) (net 33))
 (segment (start 207.01 118.11) (end 250.19 118.11) (width 0.8) (layer B.Cu) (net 33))
 (segment (start 205.74 116.84) (end 207.01 118.11) (width 0.8) (layer B.Cu) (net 33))
 (segment (start 205.74 99.695) (end 205.74 116.84) (width 0.8) (layer B.Cu) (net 33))
 (segment (start 215.265 90.17) (end 205.74 99.695) (width 0.8) (layer B.Cu) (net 33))
 (segment (start 256.54 119.38) (end 260.145001 115.774999) (width 0.8) (layer B.Cu) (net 34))
 (segment (start 260.145001 109.015001) (end 259.344999 108.214999) (width 0.8) (layer B.Cu) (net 34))
 (segment (start 260.145001 115.774999) (end 260.145001 109.015001) (width 0.8) (layer B.Cu) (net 34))
 (segment (start 259.344999 108.214999) (end 258.445 107.315) (width 0.8) (layer B.Cu) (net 34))
 (segment (start 204.47 98.425) (end 204.47 117.267071) (width 0.8) (layer B.Cu) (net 34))
 (segment (start 215.265 87.63) (end 204.47 98.425) (width 0.8) (layer B.Cu) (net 34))
 (segment (start 206.582929 119.38) (end 256.54 119.38) (width 0.8) (layer B.Cu) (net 34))
 (segment (start 204.47 117.267071) (end 206.582929 119.38) (width 0.8) (layer B.Cu) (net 34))
 (segment (start 200.025 95.25) (end 201.295 93.98) (width 0.8) (layer B.Cu) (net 6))
 (segment (start 196.85 95.25) (end 200.025 95.25) (width 0.8) (layer B.Cu) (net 6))
 (segment (start 187.96 93.98) (end 189.23 95.25) (width 0.8) (layer B.Cu) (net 41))
 (segment (start 187.96 88.9) (end 187.96 93.98) (width 0.8) (layer B.Cu) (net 41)))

